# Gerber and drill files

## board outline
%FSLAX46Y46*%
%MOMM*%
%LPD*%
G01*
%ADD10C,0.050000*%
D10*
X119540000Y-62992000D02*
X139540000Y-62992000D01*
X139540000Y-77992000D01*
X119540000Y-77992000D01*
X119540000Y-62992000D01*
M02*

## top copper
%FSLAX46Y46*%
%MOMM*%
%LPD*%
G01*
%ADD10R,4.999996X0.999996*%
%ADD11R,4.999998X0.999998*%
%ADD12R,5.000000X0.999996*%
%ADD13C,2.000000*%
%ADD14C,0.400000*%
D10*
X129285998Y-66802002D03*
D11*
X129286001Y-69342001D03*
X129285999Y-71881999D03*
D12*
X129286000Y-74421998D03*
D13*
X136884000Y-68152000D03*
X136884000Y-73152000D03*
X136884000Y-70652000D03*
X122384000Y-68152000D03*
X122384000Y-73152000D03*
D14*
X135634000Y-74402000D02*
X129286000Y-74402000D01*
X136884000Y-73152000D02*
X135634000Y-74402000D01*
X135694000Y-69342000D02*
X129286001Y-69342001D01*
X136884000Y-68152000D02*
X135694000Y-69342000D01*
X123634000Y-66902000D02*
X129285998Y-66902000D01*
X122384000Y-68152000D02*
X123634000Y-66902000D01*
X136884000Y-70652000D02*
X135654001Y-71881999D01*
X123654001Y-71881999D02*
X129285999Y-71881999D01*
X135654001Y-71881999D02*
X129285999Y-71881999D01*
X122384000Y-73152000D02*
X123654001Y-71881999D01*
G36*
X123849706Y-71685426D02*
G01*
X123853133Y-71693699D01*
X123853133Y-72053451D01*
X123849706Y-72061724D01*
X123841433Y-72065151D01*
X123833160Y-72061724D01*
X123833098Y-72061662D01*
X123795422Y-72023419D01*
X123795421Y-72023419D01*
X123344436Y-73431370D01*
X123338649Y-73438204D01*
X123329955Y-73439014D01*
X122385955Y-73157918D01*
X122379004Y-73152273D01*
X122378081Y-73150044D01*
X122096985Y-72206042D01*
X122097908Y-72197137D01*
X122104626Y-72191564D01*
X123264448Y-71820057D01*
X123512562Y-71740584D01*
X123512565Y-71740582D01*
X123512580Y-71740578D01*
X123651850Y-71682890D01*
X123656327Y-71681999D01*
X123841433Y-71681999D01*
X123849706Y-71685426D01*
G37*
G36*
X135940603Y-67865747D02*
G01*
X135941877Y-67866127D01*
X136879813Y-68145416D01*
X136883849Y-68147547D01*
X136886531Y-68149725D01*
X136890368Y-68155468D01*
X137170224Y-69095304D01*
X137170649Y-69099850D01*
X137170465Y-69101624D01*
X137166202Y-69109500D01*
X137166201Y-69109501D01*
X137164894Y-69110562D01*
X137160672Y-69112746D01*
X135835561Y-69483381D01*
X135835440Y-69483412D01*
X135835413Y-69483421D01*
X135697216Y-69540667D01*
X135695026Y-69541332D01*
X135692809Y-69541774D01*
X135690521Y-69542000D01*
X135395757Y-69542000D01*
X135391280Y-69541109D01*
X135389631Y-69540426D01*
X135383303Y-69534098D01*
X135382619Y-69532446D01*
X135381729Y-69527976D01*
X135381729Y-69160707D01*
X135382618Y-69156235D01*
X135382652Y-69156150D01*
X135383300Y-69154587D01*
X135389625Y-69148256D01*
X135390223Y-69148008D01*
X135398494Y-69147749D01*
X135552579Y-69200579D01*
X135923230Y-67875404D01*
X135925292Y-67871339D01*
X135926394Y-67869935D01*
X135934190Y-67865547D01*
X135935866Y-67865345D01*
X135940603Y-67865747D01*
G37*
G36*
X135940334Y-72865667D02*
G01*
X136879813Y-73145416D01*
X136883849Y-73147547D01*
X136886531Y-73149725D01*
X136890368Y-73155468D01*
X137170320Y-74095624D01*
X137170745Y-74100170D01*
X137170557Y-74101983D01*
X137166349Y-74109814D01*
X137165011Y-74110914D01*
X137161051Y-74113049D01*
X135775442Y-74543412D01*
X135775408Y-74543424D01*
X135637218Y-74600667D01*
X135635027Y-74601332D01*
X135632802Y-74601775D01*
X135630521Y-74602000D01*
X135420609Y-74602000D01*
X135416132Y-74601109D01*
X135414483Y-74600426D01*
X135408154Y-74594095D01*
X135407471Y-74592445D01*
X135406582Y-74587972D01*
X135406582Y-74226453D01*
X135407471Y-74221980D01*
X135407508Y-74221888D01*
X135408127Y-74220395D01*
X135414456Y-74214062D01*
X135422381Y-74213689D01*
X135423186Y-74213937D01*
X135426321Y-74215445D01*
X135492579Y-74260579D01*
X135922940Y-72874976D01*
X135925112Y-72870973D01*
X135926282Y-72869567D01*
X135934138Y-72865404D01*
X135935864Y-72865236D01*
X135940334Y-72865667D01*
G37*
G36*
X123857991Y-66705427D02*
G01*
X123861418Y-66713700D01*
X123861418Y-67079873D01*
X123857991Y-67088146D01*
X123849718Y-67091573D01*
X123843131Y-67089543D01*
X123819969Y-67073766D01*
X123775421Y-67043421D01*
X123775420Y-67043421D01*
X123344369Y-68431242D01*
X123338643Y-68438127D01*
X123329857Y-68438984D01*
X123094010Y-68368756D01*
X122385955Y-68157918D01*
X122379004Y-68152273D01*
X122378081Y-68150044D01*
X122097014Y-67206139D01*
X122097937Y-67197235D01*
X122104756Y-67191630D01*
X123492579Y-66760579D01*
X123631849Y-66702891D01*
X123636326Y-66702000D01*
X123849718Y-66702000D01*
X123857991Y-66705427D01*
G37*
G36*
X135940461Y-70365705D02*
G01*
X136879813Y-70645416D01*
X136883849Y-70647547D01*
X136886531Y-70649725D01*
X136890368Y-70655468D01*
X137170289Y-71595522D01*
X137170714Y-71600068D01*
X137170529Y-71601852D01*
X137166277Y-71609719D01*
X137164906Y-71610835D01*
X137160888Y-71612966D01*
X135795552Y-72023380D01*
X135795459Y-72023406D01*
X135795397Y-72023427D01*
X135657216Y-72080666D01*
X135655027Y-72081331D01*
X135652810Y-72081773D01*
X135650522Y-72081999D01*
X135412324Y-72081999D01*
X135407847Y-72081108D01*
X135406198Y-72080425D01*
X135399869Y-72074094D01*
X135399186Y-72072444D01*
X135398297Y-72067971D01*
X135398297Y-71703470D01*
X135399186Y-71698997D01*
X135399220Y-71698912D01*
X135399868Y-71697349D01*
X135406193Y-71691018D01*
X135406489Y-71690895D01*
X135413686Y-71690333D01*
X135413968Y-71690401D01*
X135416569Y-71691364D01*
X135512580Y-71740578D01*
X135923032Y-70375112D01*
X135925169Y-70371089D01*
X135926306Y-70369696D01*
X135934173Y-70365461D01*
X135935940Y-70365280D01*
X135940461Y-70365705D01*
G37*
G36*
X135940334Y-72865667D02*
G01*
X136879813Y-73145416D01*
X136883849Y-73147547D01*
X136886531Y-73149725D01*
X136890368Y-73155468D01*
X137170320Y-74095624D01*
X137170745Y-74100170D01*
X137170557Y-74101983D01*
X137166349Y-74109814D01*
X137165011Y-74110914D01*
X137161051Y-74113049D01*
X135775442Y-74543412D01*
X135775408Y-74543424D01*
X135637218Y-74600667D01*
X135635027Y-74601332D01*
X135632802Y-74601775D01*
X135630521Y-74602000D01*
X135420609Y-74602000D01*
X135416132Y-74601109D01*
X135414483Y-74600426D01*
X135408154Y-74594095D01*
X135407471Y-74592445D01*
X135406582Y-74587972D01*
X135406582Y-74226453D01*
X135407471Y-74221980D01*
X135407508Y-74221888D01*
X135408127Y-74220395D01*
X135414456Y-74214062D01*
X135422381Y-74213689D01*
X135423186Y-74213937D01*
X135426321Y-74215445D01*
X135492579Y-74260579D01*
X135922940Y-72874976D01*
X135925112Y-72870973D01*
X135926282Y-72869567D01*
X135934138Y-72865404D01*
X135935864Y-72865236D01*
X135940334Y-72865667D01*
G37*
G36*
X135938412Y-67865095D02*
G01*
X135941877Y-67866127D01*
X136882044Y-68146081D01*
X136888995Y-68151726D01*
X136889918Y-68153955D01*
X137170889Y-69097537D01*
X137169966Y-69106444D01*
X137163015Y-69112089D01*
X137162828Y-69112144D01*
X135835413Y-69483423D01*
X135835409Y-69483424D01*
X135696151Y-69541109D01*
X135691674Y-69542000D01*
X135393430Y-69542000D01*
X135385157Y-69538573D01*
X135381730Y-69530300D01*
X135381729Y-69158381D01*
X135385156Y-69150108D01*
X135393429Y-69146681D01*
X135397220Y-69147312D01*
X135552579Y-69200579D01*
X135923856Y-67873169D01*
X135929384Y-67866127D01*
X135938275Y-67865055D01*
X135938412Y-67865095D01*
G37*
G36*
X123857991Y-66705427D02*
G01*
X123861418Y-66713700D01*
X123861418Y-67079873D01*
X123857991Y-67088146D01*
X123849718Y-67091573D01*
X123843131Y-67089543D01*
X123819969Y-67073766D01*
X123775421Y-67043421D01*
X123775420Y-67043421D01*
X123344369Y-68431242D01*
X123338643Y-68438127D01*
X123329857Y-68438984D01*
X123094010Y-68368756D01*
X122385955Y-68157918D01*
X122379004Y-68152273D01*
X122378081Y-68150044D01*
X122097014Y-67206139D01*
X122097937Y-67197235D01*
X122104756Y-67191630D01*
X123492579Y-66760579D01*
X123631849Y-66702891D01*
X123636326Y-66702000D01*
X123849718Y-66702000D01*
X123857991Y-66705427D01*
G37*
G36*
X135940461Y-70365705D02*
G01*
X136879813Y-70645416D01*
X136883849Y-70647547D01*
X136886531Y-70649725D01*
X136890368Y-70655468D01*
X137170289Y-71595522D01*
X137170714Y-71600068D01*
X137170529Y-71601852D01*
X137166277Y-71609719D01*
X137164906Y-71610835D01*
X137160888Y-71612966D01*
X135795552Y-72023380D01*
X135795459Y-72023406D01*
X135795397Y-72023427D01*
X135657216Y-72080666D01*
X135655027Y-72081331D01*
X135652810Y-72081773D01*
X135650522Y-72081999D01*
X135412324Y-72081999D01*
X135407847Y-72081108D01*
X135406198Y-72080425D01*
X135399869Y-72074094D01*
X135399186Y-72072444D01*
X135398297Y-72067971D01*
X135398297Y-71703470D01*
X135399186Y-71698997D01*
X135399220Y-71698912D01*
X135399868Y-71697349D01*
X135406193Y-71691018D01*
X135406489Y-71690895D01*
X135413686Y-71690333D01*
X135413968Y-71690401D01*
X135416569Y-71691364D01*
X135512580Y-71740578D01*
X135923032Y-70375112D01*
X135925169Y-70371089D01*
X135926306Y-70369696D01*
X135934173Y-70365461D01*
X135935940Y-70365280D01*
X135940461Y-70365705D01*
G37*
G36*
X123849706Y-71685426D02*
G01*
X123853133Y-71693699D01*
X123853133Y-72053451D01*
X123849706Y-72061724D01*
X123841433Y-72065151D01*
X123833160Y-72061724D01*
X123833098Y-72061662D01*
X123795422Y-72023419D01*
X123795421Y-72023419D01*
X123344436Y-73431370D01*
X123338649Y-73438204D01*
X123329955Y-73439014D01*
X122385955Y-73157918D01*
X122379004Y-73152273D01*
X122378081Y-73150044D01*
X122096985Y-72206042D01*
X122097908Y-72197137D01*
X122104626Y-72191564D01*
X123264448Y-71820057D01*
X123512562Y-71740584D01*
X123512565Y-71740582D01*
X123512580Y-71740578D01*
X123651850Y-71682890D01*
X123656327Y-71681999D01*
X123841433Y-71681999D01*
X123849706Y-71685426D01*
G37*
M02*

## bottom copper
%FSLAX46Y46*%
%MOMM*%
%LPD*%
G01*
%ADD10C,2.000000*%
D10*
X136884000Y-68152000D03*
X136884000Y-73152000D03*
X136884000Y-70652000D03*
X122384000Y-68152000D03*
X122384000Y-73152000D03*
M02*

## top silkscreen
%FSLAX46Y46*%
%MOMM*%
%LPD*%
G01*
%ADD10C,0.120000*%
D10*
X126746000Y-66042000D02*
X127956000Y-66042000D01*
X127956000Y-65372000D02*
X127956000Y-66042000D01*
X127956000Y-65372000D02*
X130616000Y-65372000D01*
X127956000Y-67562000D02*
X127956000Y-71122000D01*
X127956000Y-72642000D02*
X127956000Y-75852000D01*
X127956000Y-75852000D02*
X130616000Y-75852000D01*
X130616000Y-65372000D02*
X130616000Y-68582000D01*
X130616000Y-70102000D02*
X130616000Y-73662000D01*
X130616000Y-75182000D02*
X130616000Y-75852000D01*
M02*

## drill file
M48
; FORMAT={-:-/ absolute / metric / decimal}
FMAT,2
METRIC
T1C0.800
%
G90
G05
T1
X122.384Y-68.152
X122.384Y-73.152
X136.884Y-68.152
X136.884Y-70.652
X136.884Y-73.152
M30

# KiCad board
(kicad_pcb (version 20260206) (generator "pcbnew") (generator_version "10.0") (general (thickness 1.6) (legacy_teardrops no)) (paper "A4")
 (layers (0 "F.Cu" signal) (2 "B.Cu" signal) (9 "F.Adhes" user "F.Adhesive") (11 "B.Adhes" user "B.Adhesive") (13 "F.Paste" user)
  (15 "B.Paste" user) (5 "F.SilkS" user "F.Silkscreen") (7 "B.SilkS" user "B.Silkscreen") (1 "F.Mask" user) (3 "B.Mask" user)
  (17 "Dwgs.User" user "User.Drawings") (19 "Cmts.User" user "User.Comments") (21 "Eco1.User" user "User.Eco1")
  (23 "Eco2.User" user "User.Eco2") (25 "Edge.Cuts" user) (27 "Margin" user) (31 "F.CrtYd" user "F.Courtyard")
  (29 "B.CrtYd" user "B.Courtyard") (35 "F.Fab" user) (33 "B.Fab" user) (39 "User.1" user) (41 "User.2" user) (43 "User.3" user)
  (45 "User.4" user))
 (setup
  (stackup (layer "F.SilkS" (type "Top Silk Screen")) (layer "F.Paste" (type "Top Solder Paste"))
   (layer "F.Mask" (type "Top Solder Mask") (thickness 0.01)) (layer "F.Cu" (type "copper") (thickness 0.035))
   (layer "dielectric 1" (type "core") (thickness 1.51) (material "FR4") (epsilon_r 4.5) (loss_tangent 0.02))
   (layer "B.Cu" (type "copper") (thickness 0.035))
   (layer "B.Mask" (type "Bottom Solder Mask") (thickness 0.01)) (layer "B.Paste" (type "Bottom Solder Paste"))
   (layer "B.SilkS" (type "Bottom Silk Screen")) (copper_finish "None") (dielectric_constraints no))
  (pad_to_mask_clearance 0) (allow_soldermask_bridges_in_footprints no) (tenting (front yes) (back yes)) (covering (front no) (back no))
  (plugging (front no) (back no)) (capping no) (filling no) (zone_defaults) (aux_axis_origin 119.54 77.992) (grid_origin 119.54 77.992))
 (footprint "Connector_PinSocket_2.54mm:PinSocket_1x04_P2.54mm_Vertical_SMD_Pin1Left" (layer "F.Cu") (at 129.286 70.612)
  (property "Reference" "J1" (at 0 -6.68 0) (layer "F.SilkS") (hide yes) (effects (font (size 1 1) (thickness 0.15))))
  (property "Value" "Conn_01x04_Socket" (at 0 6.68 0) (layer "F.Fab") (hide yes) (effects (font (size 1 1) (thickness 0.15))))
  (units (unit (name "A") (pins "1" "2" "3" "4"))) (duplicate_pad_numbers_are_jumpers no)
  (fp_line (start -2.54 -4.57) (end -1.33 -4.57) (stroke (width 0.12) (type solid)) (layer "F.SilkS"))
  (fp_line (start -1.33 -5.24) (end -1.33 -4.57) (stroke (width 0.12) (type solid)) (layer "F.SilkS"))
  (fp_line (start -1.33 -5.24) (end 1.33 -5.24) (stroke (width 0.12) (type solid)) (layer "F.SilkS"))
  (fp_line (start -1.33 -3.05) (end -1.33 0.51) (stroke (width 0.12) (type solid)) (layer "F.SilkS"))
  (fp_line (start -1.33 2.03) (end -1.33 5.24) (stroke (width 0.12) (type solid)) (layer "F.SilkS"))
  (fp_line (start -1.33 5.24) (end 1.33 5.24) (stroke (width 0.12) (type solid)) (layer "F.SilkS"))
  (fp_line (start 1.33 -5.24) (end 1.33 -2.03) (stroke (width 0.12) (type solid)) (layer "F.SilkS"))
  (fp_line (start 1.33 -0.51) (end 1.33 3.05) (stroke (width 0.12) (type solid)) (layer "F.SilkS"))
  (fp_line (start 1.33 4.57) (end 1.33 5.24) (stroke (width 0.12) (type solid)) (layer "F.SilkS"))
  (pad "1" smd rect (at -0.000002 -3.809998) (size 4.999996 0.999996) (layers "F.Cu" "F.Mask" "F.Paste") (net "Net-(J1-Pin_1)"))
  (pad "2" smd rect (at 0.000001 -1.269999) (size 4.999998 0.999998) (layers "F.Cu" "F.Mask" "F.Paste") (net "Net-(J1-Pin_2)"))
  (pad "3" smd rect (at -0.000001 1.269999) (size 4.999998 0.999998) (layers "F.Cu" "F.Mask" "F.Paste") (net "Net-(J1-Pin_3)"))
  (pad "4" smd rect (at 0 3.809998) (size 5 0.999996) (layers "F.Cu" "F.Mask" "F.Paste") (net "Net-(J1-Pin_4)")))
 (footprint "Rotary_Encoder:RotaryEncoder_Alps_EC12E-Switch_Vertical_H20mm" (layer "B.Cu") (at 136.884 68.152 180)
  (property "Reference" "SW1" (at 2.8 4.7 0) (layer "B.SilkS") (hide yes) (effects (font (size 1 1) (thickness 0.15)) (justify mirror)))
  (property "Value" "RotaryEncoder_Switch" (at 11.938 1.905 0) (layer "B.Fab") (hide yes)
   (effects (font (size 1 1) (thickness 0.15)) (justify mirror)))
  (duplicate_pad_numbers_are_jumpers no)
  (pad "A" thru_hole circle (at 0 0 180) (size 2 2) (drill 0.8) (layers "*.Cu" "*.Mask") (remove_unused_layers no) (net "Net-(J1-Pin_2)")
   (thermal_bridge_angle 90)
   (teardrops (best_length_ratio 0.5) (max_length 1) (best_width_ratio 1) (max_width 2) (curved_edges no) (filter_ratio 0.9) (enabled yes)
    (allow_two_segments yes) (prefer_zone_connections yes)))
  (pad "B" thru_hole circle (at 0 -5 180) (size 2 2) (drill 0.8) (layers "*.Cu" "*.Mask") (remove_unused_layers no) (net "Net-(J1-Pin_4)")
   (teardrops (best_length_ratio 0.5) (max_length 1) (best_width_ratio 1) (max_width 2) (curved_edges no) (filter_ratio 0.9) (enabled yes)
    (allow_two_segments yes) (prefer_zone_connections yes)))
  (pad "C" thru_hole circle (at 0 -2.5 180) (size 2 2) (drill 0.8) (layers "*.Cu" "*.Mask") (remove_unused_layers no) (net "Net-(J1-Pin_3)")
   (teardrops (best_length_ratio 0.5) (max_length 1) (best_width_ratio 1) (max_width 2) (curved_edges no) (filter_ratio 0.9) (enabled yes)
    (allow_two_segments yes) (prefer_zone_connections yes)))
  (pad "S1" thru_hole circle (at 14.5 0 180) (size 2 2) (drill 0.8) (layers "*.Cu" "*.Mask") (remove_unused_layers no)
   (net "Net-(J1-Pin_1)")
   (teardrops (best_length_ratio 0.5) (max_length 1) (best_width_ratio 1) (max_width 2) (curved_edges no) (filter_ratio 0.9) (enabled yes)
    (allow_two_segments yes) (prefer_zone_connections yes)))
  (pad "S2" thru_hole circle (at 14.5 -5 180) (size 2 2) (drill 0.8) (layers "*.Cu" "*.Mask") (remove_unused_layers no)
   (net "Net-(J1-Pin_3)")
   (teardrops (best_length_ratio 0.5) (max_length 1) (best_width_ratio 1) (max_width 2) (curved_edges no) (filter_ratio 0.9) (enabled yes)
    (allow_two_segments yes) (prefer_zone_connections yes))))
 (gr_rect (start 119.54 62.992) (end 139.54 77.992) (stroke (width 0.05) (type default)) (fill no) (layer "Edge.Cuts"))
 (segment (start 135.634 74.402) (end 129.286 74.402) (width 0.4) (layer "F.Cu") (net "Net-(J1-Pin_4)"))
 (segment (start 136.884 73.152) (end 135.634 74.402) (width 0.4) (layer "F.Cu") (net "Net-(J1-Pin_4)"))
 (segment (start 135.694 69.342) (end 129.286001 69.342001) (width 0.4) (layer "F.Cu") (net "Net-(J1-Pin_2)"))
 (segment (start 136.884 68.152) (end 135.694 69.342) (width 0.4) (layer "F.Cu") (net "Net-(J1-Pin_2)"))
 (segment (start 123.634 66.902) (end 129.285998 66.902) (width 0.4) (layer "F.Cu") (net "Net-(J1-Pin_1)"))
 (segment (start 122.384 68.152) (end 123.634 66.902) (width 0.4) (layer "F.Cu") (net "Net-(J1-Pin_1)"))
 (segment (start 136.884 70.652) (end 135.654001 71.881999) (width 0.4) (layer "F.Cu") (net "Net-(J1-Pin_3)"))
 (segment (start 123.654001 71.881999) (end 129.285999 71.881999) (width 0.4) (layer "F.Cu") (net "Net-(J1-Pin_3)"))
 (segment (start 135.654001 71.881999) (end 129.285999 71.881999) (width 0.4) (layer "F.Cu") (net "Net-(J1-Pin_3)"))
 (segment (start 122.384 73.152) (end 123.654001 71.881999) (width 0.4) (layer "F.Cu") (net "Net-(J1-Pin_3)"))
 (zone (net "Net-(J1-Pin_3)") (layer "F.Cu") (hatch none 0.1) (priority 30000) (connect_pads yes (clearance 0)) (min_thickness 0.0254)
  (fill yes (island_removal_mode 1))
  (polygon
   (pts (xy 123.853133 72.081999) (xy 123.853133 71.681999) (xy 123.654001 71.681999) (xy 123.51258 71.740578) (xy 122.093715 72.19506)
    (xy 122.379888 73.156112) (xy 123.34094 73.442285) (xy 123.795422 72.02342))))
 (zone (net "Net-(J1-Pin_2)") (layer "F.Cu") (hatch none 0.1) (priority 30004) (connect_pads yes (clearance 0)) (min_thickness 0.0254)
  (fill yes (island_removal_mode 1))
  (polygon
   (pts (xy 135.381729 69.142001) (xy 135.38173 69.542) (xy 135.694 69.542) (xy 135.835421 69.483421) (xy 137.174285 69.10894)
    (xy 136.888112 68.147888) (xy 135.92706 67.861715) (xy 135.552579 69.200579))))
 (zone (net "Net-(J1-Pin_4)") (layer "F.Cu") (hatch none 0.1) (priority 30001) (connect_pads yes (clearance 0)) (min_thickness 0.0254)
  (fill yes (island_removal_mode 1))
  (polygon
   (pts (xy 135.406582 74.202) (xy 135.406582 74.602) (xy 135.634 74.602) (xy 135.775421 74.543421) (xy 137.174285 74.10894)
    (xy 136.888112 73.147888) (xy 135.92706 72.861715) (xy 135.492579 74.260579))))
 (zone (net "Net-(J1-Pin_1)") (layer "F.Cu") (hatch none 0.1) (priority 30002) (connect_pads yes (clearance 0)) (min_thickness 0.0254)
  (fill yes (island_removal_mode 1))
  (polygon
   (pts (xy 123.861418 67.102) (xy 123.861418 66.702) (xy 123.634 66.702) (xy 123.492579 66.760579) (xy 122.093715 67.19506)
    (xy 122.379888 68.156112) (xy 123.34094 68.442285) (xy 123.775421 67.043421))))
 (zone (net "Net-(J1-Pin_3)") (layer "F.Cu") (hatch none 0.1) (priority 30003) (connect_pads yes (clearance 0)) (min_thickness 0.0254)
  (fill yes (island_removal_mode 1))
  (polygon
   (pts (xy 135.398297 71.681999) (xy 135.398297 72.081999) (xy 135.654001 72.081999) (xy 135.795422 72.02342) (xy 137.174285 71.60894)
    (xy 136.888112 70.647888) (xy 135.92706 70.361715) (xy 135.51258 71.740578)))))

